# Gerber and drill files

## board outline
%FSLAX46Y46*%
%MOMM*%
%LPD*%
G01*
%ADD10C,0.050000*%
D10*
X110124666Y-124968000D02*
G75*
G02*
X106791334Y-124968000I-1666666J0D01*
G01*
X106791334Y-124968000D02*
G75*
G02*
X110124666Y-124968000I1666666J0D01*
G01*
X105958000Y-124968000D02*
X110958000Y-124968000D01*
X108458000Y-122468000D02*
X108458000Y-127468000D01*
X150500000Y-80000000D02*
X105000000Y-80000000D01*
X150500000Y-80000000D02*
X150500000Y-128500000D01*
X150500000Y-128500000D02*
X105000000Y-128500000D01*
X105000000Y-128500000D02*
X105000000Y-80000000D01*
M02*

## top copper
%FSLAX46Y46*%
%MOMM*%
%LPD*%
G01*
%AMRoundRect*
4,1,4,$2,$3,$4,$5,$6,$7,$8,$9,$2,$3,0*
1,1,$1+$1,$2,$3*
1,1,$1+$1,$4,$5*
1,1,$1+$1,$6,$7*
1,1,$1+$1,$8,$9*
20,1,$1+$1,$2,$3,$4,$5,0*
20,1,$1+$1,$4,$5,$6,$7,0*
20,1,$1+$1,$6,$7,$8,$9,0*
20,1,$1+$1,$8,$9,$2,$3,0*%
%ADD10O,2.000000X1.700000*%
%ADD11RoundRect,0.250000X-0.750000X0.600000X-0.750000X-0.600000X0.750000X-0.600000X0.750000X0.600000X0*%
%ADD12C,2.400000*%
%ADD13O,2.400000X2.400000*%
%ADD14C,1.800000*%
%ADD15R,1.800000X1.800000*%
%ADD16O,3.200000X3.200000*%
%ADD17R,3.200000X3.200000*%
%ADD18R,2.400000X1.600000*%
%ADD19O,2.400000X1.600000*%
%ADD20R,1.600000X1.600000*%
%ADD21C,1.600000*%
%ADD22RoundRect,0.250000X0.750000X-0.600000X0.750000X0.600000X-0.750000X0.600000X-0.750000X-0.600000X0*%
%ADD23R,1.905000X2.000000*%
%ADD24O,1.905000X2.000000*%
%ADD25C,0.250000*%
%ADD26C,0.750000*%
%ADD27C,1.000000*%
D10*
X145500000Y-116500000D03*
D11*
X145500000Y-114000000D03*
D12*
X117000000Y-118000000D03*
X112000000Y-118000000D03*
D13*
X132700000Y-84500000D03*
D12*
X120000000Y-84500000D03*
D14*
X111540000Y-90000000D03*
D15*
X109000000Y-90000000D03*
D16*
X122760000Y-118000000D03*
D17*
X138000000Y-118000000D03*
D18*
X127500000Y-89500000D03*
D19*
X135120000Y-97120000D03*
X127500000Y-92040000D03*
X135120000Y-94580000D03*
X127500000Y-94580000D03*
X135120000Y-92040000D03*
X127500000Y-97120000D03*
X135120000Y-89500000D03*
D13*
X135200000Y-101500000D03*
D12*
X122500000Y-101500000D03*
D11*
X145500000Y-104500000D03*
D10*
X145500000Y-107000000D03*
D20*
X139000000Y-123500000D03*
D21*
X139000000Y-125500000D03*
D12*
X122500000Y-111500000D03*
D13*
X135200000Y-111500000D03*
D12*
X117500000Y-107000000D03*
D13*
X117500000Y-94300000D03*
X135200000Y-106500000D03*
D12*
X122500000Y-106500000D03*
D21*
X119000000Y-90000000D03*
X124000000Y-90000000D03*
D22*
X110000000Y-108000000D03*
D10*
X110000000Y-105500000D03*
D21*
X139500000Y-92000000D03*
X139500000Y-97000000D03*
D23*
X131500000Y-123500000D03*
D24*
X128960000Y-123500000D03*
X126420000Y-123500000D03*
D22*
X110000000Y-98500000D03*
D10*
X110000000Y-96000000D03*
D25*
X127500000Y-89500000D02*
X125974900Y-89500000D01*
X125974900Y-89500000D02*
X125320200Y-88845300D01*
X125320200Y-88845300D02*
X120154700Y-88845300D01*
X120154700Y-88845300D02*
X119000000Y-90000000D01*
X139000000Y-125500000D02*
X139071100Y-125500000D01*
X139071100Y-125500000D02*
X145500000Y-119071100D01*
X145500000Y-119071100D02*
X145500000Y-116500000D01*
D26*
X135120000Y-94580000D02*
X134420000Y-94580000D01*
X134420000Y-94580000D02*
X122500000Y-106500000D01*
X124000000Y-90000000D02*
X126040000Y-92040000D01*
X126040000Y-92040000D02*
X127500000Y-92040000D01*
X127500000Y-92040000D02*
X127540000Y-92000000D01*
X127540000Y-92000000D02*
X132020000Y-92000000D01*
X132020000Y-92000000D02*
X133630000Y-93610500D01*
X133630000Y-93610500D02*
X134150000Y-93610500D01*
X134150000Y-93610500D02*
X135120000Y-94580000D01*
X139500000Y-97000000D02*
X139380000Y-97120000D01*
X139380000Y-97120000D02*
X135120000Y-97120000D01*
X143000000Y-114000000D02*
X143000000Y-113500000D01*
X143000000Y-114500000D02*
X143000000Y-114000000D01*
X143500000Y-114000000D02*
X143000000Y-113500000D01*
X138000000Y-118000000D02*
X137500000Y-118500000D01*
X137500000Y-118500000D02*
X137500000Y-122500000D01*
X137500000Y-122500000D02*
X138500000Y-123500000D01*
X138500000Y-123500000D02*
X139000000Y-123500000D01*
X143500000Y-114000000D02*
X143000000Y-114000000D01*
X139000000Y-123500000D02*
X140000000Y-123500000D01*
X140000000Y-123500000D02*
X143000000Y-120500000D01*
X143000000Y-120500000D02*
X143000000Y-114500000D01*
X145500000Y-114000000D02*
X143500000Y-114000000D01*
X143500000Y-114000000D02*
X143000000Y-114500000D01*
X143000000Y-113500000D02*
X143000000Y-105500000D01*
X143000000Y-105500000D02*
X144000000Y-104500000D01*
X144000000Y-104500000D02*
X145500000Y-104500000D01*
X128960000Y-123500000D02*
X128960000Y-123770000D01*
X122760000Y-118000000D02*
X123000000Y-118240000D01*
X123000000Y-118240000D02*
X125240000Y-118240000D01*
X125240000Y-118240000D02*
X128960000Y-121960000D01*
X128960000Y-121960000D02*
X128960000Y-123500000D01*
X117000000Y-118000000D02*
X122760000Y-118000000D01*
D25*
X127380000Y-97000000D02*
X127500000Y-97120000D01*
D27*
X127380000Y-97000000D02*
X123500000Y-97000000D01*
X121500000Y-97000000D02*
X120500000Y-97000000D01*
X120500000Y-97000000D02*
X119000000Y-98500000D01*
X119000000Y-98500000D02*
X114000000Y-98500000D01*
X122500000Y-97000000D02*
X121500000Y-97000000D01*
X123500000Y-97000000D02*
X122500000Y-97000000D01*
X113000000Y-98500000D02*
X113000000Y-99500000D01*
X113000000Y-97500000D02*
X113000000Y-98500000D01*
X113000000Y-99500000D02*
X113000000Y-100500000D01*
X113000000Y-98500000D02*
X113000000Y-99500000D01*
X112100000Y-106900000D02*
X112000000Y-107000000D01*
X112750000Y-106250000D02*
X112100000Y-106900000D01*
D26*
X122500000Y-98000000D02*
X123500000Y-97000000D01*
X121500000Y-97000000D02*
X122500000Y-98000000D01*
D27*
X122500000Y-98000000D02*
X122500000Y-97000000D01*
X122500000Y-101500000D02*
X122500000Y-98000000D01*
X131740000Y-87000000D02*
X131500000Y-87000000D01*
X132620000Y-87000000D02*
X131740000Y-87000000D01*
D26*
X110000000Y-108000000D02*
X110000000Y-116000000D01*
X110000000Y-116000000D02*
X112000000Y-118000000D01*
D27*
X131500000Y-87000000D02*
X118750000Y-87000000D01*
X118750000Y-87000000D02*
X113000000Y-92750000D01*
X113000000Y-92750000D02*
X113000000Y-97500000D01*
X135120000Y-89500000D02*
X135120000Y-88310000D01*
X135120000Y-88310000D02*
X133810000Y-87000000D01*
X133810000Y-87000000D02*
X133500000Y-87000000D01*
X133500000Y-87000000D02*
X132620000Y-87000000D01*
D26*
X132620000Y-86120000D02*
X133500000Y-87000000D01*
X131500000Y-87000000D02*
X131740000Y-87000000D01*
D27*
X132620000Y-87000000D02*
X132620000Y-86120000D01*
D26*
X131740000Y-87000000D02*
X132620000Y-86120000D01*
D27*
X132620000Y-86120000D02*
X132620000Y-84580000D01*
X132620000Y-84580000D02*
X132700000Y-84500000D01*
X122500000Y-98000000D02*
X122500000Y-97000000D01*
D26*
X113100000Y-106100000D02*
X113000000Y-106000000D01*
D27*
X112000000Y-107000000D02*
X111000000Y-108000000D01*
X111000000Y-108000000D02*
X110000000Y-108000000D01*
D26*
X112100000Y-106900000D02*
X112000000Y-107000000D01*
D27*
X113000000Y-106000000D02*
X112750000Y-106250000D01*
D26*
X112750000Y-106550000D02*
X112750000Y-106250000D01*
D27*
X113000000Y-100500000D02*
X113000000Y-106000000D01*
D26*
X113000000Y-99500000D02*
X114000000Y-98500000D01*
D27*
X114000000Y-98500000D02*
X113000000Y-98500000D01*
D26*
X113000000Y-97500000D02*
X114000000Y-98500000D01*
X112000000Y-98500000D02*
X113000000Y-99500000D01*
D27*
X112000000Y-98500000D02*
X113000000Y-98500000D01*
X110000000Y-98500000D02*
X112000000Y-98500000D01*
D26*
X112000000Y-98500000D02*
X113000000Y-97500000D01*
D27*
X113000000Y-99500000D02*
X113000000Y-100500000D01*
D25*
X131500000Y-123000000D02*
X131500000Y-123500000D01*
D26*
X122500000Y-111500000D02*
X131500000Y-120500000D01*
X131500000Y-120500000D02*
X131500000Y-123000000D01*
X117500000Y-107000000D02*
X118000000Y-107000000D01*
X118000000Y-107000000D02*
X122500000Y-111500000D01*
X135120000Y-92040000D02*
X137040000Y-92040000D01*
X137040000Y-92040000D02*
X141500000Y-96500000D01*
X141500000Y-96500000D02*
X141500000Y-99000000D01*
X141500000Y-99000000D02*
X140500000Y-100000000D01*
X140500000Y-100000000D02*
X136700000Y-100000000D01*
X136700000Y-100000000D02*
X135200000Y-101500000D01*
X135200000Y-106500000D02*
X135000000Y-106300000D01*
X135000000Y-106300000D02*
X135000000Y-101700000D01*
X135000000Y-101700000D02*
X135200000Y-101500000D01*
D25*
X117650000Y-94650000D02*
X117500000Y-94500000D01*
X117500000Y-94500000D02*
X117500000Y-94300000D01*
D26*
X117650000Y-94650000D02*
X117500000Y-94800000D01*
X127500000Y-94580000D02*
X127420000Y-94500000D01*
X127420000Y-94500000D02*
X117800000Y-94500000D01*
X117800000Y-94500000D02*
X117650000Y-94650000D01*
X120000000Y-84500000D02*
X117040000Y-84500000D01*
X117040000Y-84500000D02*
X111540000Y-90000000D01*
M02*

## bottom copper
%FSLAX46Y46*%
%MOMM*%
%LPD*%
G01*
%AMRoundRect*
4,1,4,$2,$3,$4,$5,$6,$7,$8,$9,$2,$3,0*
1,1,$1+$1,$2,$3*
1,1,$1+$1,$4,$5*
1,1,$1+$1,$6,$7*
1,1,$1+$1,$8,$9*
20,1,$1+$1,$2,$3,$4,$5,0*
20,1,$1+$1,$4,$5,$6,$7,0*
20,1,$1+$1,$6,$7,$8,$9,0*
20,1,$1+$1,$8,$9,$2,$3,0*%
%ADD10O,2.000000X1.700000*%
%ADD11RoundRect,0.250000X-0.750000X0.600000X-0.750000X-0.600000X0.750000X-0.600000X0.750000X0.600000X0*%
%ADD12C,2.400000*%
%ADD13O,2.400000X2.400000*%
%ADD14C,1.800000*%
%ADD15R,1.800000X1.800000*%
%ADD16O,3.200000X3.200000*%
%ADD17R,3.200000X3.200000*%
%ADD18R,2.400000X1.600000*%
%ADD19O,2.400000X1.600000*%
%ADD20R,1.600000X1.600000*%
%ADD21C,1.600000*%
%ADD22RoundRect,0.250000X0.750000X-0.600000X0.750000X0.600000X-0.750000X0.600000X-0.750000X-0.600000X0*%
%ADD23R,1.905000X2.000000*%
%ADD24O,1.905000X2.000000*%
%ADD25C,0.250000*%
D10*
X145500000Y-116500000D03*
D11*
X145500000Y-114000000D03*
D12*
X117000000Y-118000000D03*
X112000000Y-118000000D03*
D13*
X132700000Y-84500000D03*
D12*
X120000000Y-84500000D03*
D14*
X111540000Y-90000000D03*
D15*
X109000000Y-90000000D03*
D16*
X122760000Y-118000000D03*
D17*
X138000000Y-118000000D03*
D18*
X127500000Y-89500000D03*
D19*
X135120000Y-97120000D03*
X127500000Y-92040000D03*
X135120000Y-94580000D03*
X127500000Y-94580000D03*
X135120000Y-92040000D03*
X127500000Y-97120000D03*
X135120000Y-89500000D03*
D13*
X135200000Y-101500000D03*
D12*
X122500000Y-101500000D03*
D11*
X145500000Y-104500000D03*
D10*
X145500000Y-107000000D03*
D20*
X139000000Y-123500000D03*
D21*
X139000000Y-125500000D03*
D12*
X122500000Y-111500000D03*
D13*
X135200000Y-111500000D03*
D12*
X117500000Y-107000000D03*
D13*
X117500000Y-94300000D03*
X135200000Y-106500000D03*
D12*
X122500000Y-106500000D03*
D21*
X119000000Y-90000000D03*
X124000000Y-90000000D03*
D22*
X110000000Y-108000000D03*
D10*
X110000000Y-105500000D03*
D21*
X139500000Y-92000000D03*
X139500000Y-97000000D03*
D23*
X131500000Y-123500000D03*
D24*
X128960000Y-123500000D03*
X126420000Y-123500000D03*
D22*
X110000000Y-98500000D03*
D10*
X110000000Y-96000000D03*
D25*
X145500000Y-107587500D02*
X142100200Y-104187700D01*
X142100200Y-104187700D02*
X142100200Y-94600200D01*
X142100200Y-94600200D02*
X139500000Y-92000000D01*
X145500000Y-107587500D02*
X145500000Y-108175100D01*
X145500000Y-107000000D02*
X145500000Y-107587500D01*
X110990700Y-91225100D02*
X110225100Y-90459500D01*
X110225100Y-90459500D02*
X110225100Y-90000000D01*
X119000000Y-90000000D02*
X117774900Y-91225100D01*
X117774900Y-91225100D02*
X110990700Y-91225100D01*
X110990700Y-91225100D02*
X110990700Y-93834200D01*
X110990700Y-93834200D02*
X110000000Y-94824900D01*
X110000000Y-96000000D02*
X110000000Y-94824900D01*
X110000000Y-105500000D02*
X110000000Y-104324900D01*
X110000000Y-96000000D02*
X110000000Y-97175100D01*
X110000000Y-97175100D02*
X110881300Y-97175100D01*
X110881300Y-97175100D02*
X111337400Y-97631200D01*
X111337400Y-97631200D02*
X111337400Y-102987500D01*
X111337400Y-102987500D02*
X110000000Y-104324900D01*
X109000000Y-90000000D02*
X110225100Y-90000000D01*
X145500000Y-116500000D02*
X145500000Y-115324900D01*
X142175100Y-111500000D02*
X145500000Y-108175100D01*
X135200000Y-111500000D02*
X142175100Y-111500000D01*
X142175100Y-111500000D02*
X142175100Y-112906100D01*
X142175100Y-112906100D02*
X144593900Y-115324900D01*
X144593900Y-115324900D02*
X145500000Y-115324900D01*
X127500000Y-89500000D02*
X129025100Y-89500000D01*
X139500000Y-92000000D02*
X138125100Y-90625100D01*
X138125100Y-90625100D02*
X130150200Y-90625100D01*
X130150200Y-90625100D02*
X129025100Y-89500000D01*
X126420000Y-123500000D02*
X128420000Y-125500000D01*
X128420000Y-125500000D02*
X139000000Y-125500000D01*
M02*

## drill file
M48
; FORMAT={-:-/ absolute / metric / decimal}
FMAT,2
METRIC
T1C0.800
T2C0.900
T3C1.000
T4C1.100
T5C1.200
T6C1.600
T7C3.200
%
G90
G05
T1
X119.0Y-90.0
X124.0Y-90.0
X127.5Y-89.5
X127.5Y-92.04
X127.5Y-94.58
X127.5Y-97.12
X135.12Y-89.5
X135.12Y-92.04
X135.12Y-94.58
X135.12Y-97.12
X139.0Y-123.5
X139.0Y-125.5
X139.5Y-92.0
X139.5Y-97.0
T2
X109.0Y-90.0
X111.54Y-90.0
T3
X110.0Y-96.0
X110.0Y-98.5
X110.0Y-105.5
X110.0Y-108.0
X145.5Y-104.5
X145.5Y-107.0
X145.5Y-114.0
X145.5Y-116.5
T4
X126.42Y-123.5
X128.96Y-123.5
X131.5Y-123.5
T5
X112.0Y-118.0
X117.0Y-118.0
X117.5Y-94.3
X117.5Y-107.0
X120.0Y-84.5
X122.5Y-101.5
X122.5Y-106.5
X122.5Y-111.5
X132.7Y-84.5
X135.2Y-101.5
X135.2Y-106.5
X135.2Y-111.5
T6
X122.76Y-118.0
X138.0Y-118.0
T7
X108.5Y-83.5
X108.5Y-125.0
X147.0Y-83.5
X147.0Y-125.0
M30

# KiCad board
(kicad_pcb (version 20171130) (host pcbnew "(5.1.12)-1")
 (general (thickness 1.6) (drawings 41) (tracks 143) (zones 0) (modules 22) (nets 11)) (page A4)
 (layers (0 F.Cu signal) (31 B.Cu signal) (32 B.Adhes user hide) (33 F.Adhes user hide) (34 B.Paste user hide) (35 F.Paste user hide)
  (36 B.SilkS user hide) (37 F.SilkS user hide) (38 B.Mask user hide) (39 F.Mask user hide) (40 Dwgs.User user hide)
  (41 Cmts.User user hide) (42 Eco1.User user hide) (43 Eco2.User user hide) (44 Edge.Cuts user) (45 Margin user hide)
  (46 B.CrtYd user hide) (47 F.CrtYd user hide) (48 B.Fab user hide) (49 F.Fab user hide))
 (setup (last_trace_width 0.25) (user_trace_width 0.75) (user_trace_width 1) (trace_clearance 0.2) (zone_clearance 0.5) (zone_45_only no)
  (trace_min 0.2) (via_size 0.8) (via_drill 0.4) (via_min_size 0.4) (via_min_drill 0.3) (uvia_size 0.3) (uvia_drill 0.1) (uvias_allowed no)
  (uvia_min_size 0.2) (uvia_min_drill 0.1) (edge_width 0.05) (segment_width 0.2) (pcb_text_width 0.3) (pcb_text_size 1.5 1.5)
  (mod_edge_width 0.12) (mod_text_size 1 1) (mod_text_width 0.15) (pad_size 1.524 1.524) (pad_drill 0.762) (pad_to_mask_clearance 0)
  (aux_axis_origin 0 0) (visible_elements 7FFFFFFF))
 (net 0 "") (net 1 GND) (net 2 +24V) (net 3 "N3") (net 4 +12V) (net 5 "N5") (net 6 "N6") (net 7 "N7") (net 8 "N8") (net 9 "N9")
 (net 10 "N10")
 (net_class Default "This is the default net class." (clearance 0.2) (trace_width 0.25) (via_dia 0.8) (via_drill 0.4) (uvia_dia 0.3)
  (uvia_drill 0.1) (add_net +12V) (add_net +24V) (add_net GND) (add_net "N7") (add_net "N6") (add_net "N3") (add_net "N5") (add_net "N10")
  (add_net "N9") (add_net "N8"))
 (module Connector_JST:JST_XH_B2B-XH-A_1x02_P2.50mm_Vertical (layer F.Cu) (at 145.5 114 270)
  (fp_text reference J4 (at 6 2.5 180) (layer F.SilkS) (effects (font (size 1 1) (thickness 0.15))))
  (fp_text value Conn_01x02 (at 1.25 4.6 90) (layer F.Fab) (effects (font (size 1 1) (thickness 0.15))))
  (pad 2 thru_hole oval (at 2.5 0 270) (size 1.7 2) (drill 1) (layers *.Cu *.Mask) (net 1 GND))
  (pad 1 thru_hole roundrect (at 0 0 270) (size 1.7 2) (drill 1) (layers *.Cu *.Mask) (roundrect_rratio 0.1470588235294118) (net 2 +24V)))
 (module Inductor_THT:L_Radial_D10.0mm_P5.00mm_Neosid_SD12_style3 (layer F.Cu) (at 112 118)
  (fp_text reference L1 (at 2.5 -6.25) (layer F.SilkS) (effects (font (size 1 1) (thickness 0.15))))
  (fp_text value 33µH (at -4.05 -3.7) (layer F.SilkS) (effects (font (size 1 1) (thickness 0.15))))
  (pad 2 thru_hole circle (at 5 0) (size 2.4 2.4) (drill 1.2) (layers *.Cu *.Mask) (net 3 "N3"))
  (pad 1 thru_hole circle (at 0 0) (size 2.4 2.4) (drill 1.2) (layers *.Cu *.Mask) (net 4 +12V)))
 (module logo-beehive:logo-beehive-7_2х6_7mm (layer F.Cu) (at 139 85)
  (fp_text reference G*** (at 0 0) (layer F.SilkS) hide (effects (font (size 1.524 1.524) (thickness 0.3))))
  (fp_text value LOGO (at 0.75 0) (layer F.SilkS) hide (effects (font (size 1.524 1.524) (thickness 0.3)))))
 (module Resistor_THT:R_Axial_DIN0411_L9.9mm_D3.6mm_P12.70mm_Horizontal (layer F.Cu) (at 120 84.5)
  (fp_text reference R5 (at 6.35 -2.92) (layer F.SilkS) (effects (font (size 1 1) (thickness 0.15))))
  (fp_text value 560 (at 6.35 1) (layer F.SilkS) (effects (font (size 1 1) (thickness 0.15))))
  (pad 2 thru_hole oval (at 12.7 0) (size 2.4 2.4) (drill 1.2) (layers *.Cu *.Mask) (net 4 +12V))
  (pad 1 thru_hole circle (at 0 0) (size 2.4 2.4) (drill 1.2) (layers *.Cu *.Mask) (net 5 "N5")))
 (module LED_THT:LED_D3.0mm (layer F.Cu) (at 109 90)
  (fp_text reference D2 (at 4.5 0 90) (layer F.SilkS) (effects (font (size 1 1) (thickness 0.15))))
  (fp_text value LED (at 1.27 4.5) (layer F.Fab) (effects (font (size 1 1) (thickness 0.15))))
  (pad 2 thru_hole circle (at 2.54 0) (size 1.8 1.8) (drill 0.9) (layers *.Cu *.Mask) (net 5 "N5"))
  (pad 1 thru_hole rect (at 0 0) (size 1.8 1.8) (drill 0.9) (layers *.Cu *.Mask) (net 1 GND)))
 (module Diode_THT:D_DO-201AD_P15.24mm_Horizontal (layer F.Cu) (at 138 118 180)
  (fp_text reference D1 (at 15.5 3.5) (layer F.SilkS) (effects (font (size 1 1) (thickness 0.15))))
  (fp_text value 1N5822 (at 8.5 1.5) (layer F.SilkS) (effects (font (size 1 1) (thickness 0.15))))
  (pad 2 thru_hole oval (at 15.24 0 180) (size 3.2 3.2) (drill 1.6) (layers *.Cu *.Mask) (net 3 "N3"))
  (pad 1 thru_hole rect (at 0 0 180) (size 3.2 3.2) (drill 1.6) (layers *.Cu *.Mask) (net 2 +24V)))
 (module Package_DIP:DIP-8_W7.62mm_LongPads (layer F.Cu) (at 127.5 89.5)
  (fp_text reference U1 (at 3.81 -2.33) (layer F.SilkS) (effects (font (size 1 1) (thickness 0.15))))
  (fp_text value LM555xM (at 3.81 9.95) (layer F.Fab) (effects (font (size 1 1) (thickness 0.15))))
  (pad 1 thru_hole rect (at 0 0) (size 2.4 1.6) (drill 0.8) (layers *.Cu *.Mask) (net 1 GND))
  (pad 5 thru_hole oval (at 7.62 7.62) (size 2.4 1.6) (drill 0.8) (layers *.Cu *.Mask) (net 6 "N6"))
  (pad 2 thru_hole oval (at 0 2.54) (size 2.4 1.6) (drill 0.8) (layers *.Cu *.Mask) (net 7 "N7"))
  (pad 6 thru_hole oval (at 7.62 5.08) (size 2.4 1.6) (drill 0.8) (layers *.Cu *.Mask) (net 7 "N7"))
  (pad 3 thru_hole oval (at 0 5.08) (size 2.4 1.6) (drill 0.8) (layers *.Cu *.Mask) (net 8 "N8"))
  (pad 7 thru_hole oval (at 7.62 2.54) (size 2.4 1.6) (drill 0.8) (layers *.Cu *.Mask) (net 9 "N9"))
  (pad 4 thru_hole oval (at 0 7.62) (size 2.4 1.6) (drill 0.8) (layers *.Cu *.Mask) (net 4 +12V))
  (pad 8 thru_hole oval (at 7.62 0) (size 2.4 1.6) (drill 0.8) (layers *.Cu *.Mask) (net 4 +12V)))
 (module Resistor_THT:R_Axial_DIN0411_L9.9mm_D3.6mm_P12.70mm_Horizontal (layer F.Cu) (at 122.5 101.5)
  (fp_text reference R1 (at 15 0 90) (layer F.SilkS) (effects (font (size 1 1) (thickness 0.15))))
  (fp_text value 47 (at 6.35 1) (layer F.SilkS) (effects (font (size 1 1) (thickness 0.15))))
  (pad 2 thru_hole oval (at 12.7 0) (size 2.4 2.4) (drill 1.2) (layers *.Cu *.Mask) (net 9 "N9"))
  (pad 1 thru_hole circle (at 0 0) (size 2.4 2.4) (drill 1.2) (layers *.Cu *.Mask) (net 4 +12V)))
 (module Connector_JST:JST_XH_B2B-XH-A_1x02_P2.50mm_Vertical (layer F.Cu) (at 145.5 104.5 270)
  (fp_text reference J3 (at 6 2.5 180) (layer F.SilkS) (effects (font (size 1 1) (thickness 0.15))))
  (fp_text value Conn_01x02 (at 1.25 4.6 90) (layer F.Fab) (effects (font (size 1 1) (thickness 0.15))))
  (pad 1 thru_hole roundrect (at 0 0 270) (size 1.7 2) (drill 1) (layers *.Cu *.Mask) (roundrect_rratio 0.1470588235294118) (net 2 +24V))
  (pad 2 thru_hole oval (at 2.5 0 270) (size 1.7 2) (drill 1) (layers *.Cu *.Mask) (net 1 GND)))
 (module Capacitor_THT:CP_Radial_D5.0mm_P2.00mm (layer F.Cu) (at 139 123.5 270)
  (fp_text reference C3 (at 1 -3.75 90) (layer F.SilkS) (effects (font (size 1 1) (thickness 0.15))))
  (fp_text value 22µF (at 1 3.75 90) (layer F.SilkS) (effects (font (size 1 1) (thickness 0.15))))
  (pad 1 thru_hole rect (at 0 0 270) (size 1.6 1.6) (drill 0.8) (layers *.Cu *.Mask) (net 2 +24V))
  (pad 2 thru_hole circle (at 2 0 270) (size 1.6 1.6) (drill 0.8) (layers *.Cu *.Mask) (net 1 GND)))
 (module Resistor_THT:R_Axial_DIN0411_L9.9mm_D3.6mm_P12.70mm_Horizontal (layer F.Cu) (at 122.5 111.5)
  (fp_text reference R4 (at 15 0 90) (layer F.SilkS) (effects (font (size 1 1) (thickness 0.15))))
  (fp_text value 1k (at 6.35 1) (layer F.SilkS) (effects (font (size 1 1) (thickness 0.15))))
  (pad 1 thru_hole circle (at 0 0) (size 2.4 2.4) (drill 1.2) (layers *.Cu *.Mask) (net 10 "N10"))
  (pad 2 thru_hole oval (at 12.7 0) (size 2.4 2.4) (drill 1.2) (layers *.Cu *.Mask) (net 1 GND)))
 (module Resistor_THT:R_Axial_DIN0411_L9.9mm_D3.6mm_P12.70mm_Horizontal (layer F.Cu) (at 117.5 107 90)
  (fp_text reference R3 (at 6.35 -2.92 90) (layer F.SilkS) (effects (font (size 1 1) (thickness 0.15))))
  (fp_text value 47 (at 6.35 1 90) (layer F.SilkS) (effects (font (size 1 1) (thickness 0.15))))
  (pad 1 thru_hole circle (at 0 0 90) (size 2.4 2.4) (drill 1.2) (layers *.Cu *.Mask) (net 10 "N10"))
  (pad 2 thru_hole oval (at 12.7 0 90) (size 2.4 2.4) (drill 1.2) (layers *.Cu *.Mask) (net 8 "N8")))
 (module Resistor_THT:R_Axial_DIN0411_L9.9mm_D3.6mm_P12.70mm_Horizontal (layer F.Cu) (at 122.5 106.5)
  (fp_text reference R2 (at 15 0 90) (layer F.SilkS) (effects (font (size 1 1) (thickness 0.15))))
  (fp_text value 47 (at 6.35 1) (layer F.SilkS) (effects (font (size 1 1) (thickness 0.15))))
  (pad 2 thru_hole oval (at 12.7 0) (size 2.4 2.4) (drill 1.2) (layers *.Cu *.Mask) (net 9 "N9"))
  (pad 1 thru_hole circle (at 0 0) (size 2.4 2.4) (drill 1.2) (layers *.Cu *.Mask) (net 7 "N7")))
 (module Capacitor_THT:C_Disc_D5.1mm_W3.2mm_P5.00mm (layer F.Cu) (at 119 90)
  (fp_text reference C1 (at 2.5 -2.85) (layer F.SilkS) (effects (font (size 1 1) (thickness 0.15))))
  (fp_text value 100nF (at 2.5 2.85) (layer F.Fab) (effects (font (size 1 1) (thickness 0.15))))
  (pad 1 thru_hole circle (at 0 0) (size 1.6 1.6) (drill 0.8) (layers *.Cu *.Mask) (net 1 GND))
  (pad 2 thru_hole circle (at 5 0) (size 1.6 1.6) (drill 0.8) (layers *.Cu *.Mask) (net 7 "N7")))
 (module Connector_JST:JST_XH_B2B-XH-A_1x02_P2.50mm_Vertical (layer F.Cu) (at 110 108 90)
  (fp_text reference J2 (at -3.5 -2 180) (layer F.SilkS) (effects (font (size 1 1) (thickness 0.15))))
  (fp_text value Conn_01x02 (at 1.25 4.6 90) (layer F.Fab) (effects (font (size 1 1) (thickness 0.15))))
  (pad 1 thru_hole roundrect (at 0 0 90) (size 1.7 2) (drill 1) (layers *.Cu *.Mask) (roundrect_rratio 0.1470588235294118) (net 4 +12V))
  (pad 2 thru_hole oval (at 2.5 0 90) (size 1.7 2) (drill 1) (layers *.Cu *.Mask) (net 1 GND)))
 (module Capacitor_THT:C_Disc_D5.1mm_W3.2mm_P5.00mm (layer F.Cu) (at 139.5 92 270)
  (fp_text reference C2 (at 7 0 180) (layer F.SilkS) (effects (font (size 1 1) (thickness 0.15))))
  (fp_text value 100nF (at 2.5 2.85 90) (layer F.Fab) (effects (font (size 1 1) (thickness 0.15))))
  (pad 1 thru_hole circle (at 0 0 270) (size 1.6 1.6) (drill 0.8) (layers *.Cu *.Mask) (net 1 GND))
  (pad 2 thru_hole circle (at 5 0 270) (size 1.6 1.6) (drill 0.8) (layers *.Cu *.Mask) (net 6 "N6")))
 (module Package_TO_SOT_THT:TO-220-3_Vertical (layer F.Cu) (at 131.5 123.5 180)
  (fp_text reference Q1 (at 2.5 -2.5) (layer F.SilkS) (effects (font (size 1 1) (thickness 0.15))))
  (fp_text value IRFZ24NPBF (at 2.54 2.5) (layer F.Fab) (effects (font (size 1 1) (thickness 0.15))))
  (pad 1 thru_hole rect (at 0 0 180) (size 1.905 2) (drill 1.1) (layers *.Cu *.Mask) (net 10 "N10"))
  (pad 2 thru_hole oval (at 2.54 0 180) (size 1.905 2) (drill 1.1) (layers *.Cu *.Mask) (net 3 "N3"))
  (pad 3 thru_hole oval (at 5.08 0 180) (size 1.905 2) (drill 1.1) (layers *.Cu *.Mask) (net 1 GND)))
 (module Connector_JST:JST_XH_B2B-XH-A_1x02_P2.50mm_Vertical (layer F.Cu) (at 110 98.5 90)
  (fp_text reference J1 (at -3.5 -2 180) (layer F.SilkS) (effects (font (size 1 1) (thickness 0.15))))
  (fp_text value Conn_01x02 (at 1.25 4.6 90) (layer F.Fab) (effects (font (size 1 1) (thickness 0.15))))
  (pad 1 thru_hole roundrect (at 0 0 90) (size 1.7 2) (drill 1) (layers *.Cu *.Mask) (roundrect_rratio 0.1470588235294118) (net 4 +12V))
  (pad 2 thru_hole oval (at 2.5 0 90) (size 1.7 2) (drill 1) (layers *.Cu *.Mask) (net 1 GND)))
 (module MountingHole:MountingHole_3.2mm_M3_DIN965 (layer F.Cu) (at 147 83.5)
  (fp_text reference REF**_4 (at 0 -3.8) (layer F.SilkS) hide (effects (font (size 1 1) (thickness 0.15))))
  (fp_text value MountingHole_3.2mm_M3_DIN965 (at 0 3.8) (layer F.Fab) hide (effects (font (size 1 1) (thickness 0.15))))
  (pad 1 np_thru_hole circle (at 0 0) (size 3.2 3.2) (drill 3.2) (layers *.Cu *.Mask)))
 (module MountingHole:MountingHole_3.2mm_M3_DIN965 (layer F.Cu) (at 108.5 125)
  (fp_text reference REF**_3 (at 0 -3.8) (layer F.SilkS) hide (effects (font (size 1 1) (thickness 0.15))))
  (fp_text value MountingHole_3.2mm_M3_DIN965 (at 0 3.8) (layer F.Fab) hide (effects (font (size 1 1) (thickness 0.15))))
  (pad 1 np_thru_hole circle (at 0 0) (size 3.2 3.2) (drill 3.2) (layers *.Cu *.Mask)))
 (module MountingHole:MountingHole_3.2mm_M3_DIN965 (layer F.Cu) (at 147 125)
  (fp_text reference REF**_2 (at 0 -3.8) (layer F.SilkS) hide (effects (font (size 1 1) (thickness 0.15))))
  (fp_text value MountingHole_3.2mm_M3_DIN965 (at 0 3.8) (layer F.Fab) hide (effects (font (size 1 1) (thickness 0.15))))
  (pad 1 np_thru_hole circle (at 0 0) (size 3.2 3.2) (drill 3.2) (layers *.Cu *.Mask)))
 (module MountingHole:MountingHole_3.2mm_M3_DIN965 (layer F.Cu) (at 108.5 83.5)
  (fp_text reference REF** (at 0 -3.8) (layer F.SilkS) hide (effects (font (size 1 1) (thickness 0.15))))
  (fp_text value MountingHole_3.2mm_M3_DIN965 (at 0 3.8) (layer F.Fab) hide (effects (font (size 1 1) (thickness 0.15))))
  (pad 1 np_thru_hole circle (at 0 0) (size 3.2 3.2) (drill 3.2) (layers *.Cu *.Mask)))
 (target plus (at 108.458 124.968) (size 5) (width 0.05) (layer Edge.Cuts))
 (gr_line (start 150.5 80) (end 105 80) (layer Edge.Cuts) (width 0.05))
 (gr_line (start 150.5 80) (end 150.5 128.5) (layer Edge.Cuts) (width 0.05))
 (gr_line (start 150.5 128.5) (end 105 128.5) (layer Edge.Cuts) (width 0.05))
 (gr_line (start 105 128.5) (end 105 80) (layer Edge.Cuts) (width 0.05))
 (segment (start 145.5 107.5875) (end 142.1002 104.1877) (width 0.25) (layer B.Cu) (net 1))
 (segment (start 142.1002 104.1877) (end 142.1002 94.6002) (width 0.25) (layer B.Cu) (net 1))
 (segment (start 142.1002 94.6002) (end 139.5 92) (width 0.25) (layer B.Cu) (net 1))
 (segment (start 145.5 107.5875) (end 145.5 108.1751) (width 0.25) (layer B.Cu) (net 1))
 (segment (start 145.5 107) (end 145.5 107.5875) (width 0.25) (layer B.Cu) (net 1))
 (segment (start 127.5 89.5) (end 125.9749 89.5) (width 0.25) (layer F.Cu) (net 1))
 (segment (start 125.9749 89.5) (end 125.3202 88.8453) (width 0.25) (layer F.Cu) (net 1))
 (segment (start 125.3202 88.8453) (end 120.1547 88.8453) (width 0.25) (layer F.Cu) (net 1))
 (segment (start 120.1547 88.8453) (end 119 90) (width 0.25) (layer F.Cu) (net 1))
 (segment (start 110.9907 91.2251) (end 110.2251 90.4595) (width 0.25) (layer B.Cu) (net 1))
 (segment (start 110.2251 90.4595) (end 110.2251 90) (width 0.25) (layer B.Cu) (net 1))
 (segment (start 119 90) (end 117.7749 91.2251) (width 0.25) (layer B.Cu) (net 1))
 (segment (start 117.7749 91.2251) (end 110.9907 91.2251) (width 0.25) (layer B.Cu) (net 1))
 (segment (start 110.9907 91.2251) (end 110.9907 93.8342) (width 0.25) (layer B.Cu) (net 1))
 (segment (start 110.9907 93.8342) (end 110 94.8249) (width 0.25) (layer B.Cu) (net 1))
 (segment (start 110 96) (end 110 94.8249) (width 0.25) (layer B.Cu) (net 1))
 (segment (start 110 105.5) (end 110 104.3249) (width 0.25) (layer B.Cu) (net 1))
 (segment (start 110 96) (end 110 97.1751) (width 0.25) (layer B.Cu) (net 1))
 (segment (start 110 97.1751) (end 110.8813 97.1751) (width 0.25) (layer B.Cu) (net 1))
 (segment (start 110.8813 97.1751) (end 111.3374 97.6312) (width 0.25) (layer B.Cu) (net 1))
 (segment (start 111.3374 97.6312) (end 111.3374 102.9875) (width 0.25) (layer B.Cu) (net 1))
 (segment (start 111.3374 102.9875) (end 110 104.3249) (width 0.25) (layer B.Cu) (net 1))
 (segment (start 109 90) (end 110.2251 90) (width 0.25) (layer B.Cu) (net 1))
 (segment (start 145.5 116.5) (end 145.5 115.3249) (width 0.25) (layer B.Cu) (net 1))
 (segment (start 142.1751 111.5) (end 145.5 108.1751) (width 0.25) (layer B.Cu) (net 1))
 (segment (start 135.2 111.5) (end 142.1751 111.5) (width 0.25) (layer B.Cu) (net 1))
 (segment (start 142.1751 111.5) (end 142.1751 112.9061) (width 0.25) (layer B.Cu) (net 1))
 (segment (start 142.1751 112.9061) (end 144.5939 115.3249) (width 0.25) (layer B.Cu) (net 1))
 (segment (start 144.5939 115.3249) (end 145.5 115.3249) (width 0.25) (layer B.Cu) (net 1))
 (segment (start 139 125.5) (end 139.0711 125.5) (width 0.25) (layer F.Cu) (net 1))
 (segment (start 139.0711 125.5) (end 145.5 119.0711) (width 0.25) (layer F.Cu) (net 1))
 (segment (start 145.5 119.0711) (end 145.5 116.5) (width 0.25) (layer F.Cu) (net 1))
 (segment (start 127.5 89.5) (end 129.0251 89.5) (width 0.25) (layer B.Cu) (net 1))
 (segment (start 139.5 92) (end 138.1251 90.6251) (width 0.25) (layer B.Cu) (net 1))
 (segment (start 138.1251 90.6251) (end 130.1502 90.6251) (width 0.25) (layer B.Cu) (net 1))
 (segment (start 130.1502 90.6251) (end 129.0251 89.5) (width 0.25) (layer B.Cu) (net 1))
 (segment (start 126.42 123.5) (end 128.42 125.5) (width 0.25) (layer B.Cu) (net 1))
 (segment (start 128.42 125.5) (end 139 125.5) (width 0.25) (layer B.Cu) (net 1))
 (segment (start 135.12 94.58) (end 134.42 94.58) (width 0.75) (layer F.Cu) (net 7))
 (segment (start 134.42 94.58) (end 122.5 106.5) (width 0.75) (layer F.Cu) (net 7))
 (segment (start 124 90) (end 126.04 92.04) (width 0.75) (layer F.Cu) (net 7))
 (segment (start 126.04 92.04) (end 127.5 92.04) (width 0.75) (layer F.Cu) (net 7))
 (segment (start 127.5 92.04) (end 127.54 92) (width 0.75) (layer F.Cu) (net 7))
 (segment (start 127.54 92) (end 132.02 92) (width 0.75) (layer F.Cu) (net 7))
 (segment (start 132.02 92) (end 133.63 93.6105) (width 0.75) (layer F.Cu) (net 7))
 (segment (start 133.63 93.6105) (end 134.15 93.6105) (width 0.75) (layer F.Cu) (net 7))
 (segment (start 134.15 93.6105) (end 135.12 94.58) (width 0.75) (layer F.Cu) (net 7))
 (segment (start 139.5 97) (end 139.38 97.12) (width 0.75) (layer F.Cu) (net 6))
 (segment (start 139.38 97.12) (end 135.12 97.12) (width 0.75) (layer F.Cu) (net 6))
 (segment (start 143 114) (end 143 113.5) (width 0.75) (layer F.Cu) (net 2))
 (segment (start 143 114.5) (end 143 114) (width 0.75) (layer F.Cu) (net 2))
 (segment (start 143.5 114) (end 143 113.5) (width 0.75) (layer F.Cu) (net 2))
 (segment (start 138 118) (end 137.5 118.5) (width 0.75) (layer F.Cu) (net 2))
 (segment (start 137.5 118.5) (end 137.5 122.5) (width 0.75) (layer F.Cu) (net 2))
 (segment (start 137.5 122.5) (end 138.5 123.5) (width 0.75) (layer F.Cu) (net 2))
 (segment (start 138.5 123.5) (end 139 123.5) (width 0.75) (layer F.Cu) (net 2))
 (segment (start 143.5 114) (end 143 114) (width 0.75) (layer F.Cu) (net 2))
 (segment (start 139 123.5) (end 140 123.5) (width 0.75) (layer F.Cu) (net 2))
 (segment (start 140 123.5) (end 143 120.5) (width 0.75) (layer F.Cu) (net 2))
 (segment (start 143 120.5) (end 143 114.5) (width 0.75) (layer F.Cu) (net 2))
 (segment (start 145.5 114) (end 143.5 114) (width 0.75) (layer F.Cu) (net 2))
 (segment (start 143.5 114) (end 143 114.5) (width 0.75) (layer F.Cu) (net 2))
 (segment (start 143 113.5) (end 143 105.5) (width 0.75) (layer F.Cu) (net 2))
 (segment (start 143 105.5) (end 144 104.5) (width 0.75) (layer F.Cu) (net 2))
 (segment (start 144 104.5) (end 145.5 104.5) (width 0.75) (layer F.Cu) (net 2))
 (segment (start 128.96 123.5) (end 128.96 123.77) (width 0.75) (layer F.Cu) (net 3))
 (segment (start 122.76 118) (end 123 118.24) (width 0.75) (layer F.Cu) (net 3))
 (segment (start 123 118.24) (end 125.24 118.24) (width 0.75) (layer F.Cu) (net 3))
 (segment (start 125.24 118.24) (end 128.96 121.96) (width 0.75) (layer F.Cu) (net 3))
 (segment (start 128.96 121.96) (end 128.96 123.5) (width 0.75) (layer F.Cu) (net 3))
 (segment (start 117 118) (end 122.76 118) (width 0.75) (layer F.Cu) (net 3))
 (segment (start 127.38 97) (end 127.5 97.12) (width 0.25) (layer F.Cu) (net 4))
 (segment (start 127.38 97) (end 123.5 97) (width 1) (layer F.Cu) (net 4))
 (segment (start 121.5 97) (end 120.5 97) (width 1) (layer F.Cu) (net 4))
 (segment (start 120.5 97) (end 119 98.5) (width 1) (layer F.Cu) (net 4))
 (segment (start 119 98.5) (end 114 98.5) (width 1) (layer F.Cu) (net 4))
 (segment (start 122.5 97) (end 121.5 97) (width 1) (layer F.Cu) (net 4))
 (segment (start 123.5 97) (end 122.5 97) (width 1) (layer F.Cu) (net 4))
 (segment (start 113 98.5) (end 113 99.5) (width 1) (layer F.Cu) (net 4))
 (segment (start 113 97.5) (end 113 98.5) (width 1) (layer F.Cu) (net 4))
 (segment (start 113 99.5) (end 113 100.5) (width 1) (layer F.Cu) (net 4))
 (segment (start 113 98.5) (end 113 99.5) (width 1) (layer F.Cu) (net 4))
 (segment (start 112.1 106.9) (end 112 107) (width 1) (layer F.Cu) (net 4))
 (segment (start 112.75 106.25) (end 112.1 106.9) (width 1) (layer F.Cu) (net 4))
 (segment (start 122.5 98) (end 123.5 97) (width 0.75) (layer F.Cu) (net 4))
 (segment (start 121.5 97) (end 122.5 98) (width 0.75) (layer F.Cu) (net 4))
 (segment (start 122.5 98) (end 122.5 97) (width 1) (layer F.Cu) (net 4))
 (segment (start 122.5 101.5) (end 122.5 98) (width 1) (layer F.Cu) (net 4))
 (segment (start 131.74 87) (end 131.5 87) (width 1) (layer F.Cu) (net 4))
 (segment (start 132.62 87) (end 131.74 87) (width 1) (layer F.Cu) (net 4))
 (segment (start 110 108) (end 110 116) (width 0.75) (layer F.Cu) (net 4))
 (segment (start 110 116) (end 112 118) (width 0.75) (layer F.Cu) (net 4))
 (segment (start 131.5 87) (end 118.75 87) (width 1) (layer F.Cu) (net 4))
 (segment (start 118.75 87) (end 113 92.75) (width 1) (layer F.Cu) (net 4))
 (segment (start 113 92.75) (end 113 97.5) (width 1) (layer F.Cu) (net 4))
 (segment (start 135.12 89.5) (end 135.12 88.31) (width 1) (layer F.Cu) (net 4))
 (segment (start 135.12 88.31) (end 133.81 87) (width 1) (layer F.Cu) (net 4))
 (segment (start 133.81 87) (end 133.5 87) (width 1) (layer F.Cu) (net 4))
 (segment (start 133.5 87) (end 132.62 87) (width 1) (layer F.Cu) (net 4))
 (segment (start 132.62 86.12) (end 133.5 87) (width 0.75) (layer F.Cu) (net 4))
 (segment (start 131.5 87) (end 131.74 87) (width 0.75) (layer F.Cu) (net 4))
 (segment (start 132.62 87) (end 132.62 86.12) (width 1) (layer F.Cu) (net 4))
 (segment (start 131.74 87) (end 132.62 86.12) (width 0.75) (layer F.Cu) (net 4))
 (segment (start 132.62 86.12) (end 132.62 84.58) (width 1) (layer F.Cu) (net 4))
 (segment (start 132.62 84.58) (end 132.7 84.5) (width 1) (layer F.Cu) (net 4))
 (segment (start 122.5 98) (end 122.5 97) (width 1) (layer F.Cu) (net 4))
 (segment (start 113.1 106.1) (end 113 106) (width 0.75) (layer F.Cu) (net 4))
 (segment (start 112 107) (end 111 108) (width 1) (layer F.Cu) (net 4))
 (segment (start 111 108) (end 110 108) (width 1) (layer F.Cu) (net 4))
 (segment (start 112.1 106.9) (end 112 107) (width 0.75) (layer F.Cu) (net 4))
 (segment (start 113 106) (end 112.75 106.25) (width 1) (layer F.Cu) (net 4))
 (segment (start 112.75 106.55) (end 112.75 106.25) (width 0.75) (layer F.Cu) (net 4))
 (segment (start 113 100.5) (end 113 106) (width 1) (layer F.Cu) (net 4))
 (segment (start 113 99.5) (end 114 98.5) (width 0.75) (layer F.Cu) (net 4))
 (segment (start 114 98.5) (end 113 98.5) (width 1) (layer F.Cu) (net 4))
 (segment (start 113 97.5) (end 114 98.5) (width 0.75) (layer F.Cu) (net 4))
 (segment (start 112 98.5) (end 113 99.5) (width 0.75) (layer F.Cu) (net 4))
 (segment (start 112 98.5) (end 113 98.5) (width 1) (layer F.Cu) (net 4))
 (segment (start 110 98.5) (end 112 98.5) (width 1) (layer F.Cu) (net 4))
 (segment (start 112 98.5) (end 113 97.5) (width 0.75) (layer F.Cu) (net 4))
 (segment (start 113 99.5) (end 113 100.5) (width 1) (layer F.Cu) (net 4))
 (segment (start 131.5 123) (end 131.5 123.5) (width 0.25) (layer F.Cu) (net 10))
 (segment (start 122.5 111.5) (end 131.5 120.5) (width 0.75) (layer F.Cu) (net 10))
 (segment (start 131.5 120.5) (end 131.5 123) (width 0.75) (layer F.Cu) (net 10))
 (segment (start 117.5 107) (end 118 107) (width 0.75) (layer F.Cu) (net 10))
 (segment (start 118 107) (end 122.5 111.5) (width 0.75) (layer F.Cu) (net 10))
 (segment (start 135.12 92.04) (end 137.04 92.04) (width 0.75) (layer F.Cu) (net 9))
 (segment (start 137.04 92.04) (end 141.5 96.5) (width 0.75) (layer F.Cu) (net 9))
 (segment (start 141.5 96.5) (end 141.5 99) (width 0.75) (layer F.Cu) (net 9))
 (segment (start 141.5 99) (end 140.5 100) (width 0.75) (layer F.Cu) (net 9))
 (segment (start 140.5 100) (end 136.7 100) (width 0.75) (layer F.Cu) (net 9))
 (segment (start 136.7 100) (end 135.2 101.5) (width 0.75) (layer F.Cu) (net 9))
 (segment (start 135.2 106.5) (end 135 106.3) (width 0.75) (layer F.Cu) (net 9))
 (segment (start 135 106.3) (end 135 101.7) (width 0.75) (layer F.Cu) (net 9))
 (segment (start 135 101.7) (end 135.2 101.5) (width 0.75) (layer F.Cu) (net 9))
 (segment (start 117.65 94.65) (end 117.5 94.5) (width 0.25) (layer F.Cu) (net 8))
 (segment (start 117.5 94.5) (end 117.5 94.3) (width 0.25) (layer F.Cu) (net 8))
 (segment (start 117.65 94.65) (end 117.5 94.8) (width 0.75) (layer F.Cu) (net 8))
 (segment (start 127.5 94.58) (end 127.42 94.5) (width 0.75) (layer F.Cu) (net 8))
 (segment (start 127.42 94.5) (end 117.8 94.5) (width 0.75) (layer F.Cu) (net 8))
 (segment (start 117.8 94.5) (end 117.65 94.65) (width 0.75) (layer F.Cu) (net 8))
 (segment (start 120 84.5) (end 117.04 84.5) (width 0.75) (layer F.Cu) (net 5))
 (segment (start 117.04 84.5) (end 111.54 90) (width 0.75) (layer F.Cu) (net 5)))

